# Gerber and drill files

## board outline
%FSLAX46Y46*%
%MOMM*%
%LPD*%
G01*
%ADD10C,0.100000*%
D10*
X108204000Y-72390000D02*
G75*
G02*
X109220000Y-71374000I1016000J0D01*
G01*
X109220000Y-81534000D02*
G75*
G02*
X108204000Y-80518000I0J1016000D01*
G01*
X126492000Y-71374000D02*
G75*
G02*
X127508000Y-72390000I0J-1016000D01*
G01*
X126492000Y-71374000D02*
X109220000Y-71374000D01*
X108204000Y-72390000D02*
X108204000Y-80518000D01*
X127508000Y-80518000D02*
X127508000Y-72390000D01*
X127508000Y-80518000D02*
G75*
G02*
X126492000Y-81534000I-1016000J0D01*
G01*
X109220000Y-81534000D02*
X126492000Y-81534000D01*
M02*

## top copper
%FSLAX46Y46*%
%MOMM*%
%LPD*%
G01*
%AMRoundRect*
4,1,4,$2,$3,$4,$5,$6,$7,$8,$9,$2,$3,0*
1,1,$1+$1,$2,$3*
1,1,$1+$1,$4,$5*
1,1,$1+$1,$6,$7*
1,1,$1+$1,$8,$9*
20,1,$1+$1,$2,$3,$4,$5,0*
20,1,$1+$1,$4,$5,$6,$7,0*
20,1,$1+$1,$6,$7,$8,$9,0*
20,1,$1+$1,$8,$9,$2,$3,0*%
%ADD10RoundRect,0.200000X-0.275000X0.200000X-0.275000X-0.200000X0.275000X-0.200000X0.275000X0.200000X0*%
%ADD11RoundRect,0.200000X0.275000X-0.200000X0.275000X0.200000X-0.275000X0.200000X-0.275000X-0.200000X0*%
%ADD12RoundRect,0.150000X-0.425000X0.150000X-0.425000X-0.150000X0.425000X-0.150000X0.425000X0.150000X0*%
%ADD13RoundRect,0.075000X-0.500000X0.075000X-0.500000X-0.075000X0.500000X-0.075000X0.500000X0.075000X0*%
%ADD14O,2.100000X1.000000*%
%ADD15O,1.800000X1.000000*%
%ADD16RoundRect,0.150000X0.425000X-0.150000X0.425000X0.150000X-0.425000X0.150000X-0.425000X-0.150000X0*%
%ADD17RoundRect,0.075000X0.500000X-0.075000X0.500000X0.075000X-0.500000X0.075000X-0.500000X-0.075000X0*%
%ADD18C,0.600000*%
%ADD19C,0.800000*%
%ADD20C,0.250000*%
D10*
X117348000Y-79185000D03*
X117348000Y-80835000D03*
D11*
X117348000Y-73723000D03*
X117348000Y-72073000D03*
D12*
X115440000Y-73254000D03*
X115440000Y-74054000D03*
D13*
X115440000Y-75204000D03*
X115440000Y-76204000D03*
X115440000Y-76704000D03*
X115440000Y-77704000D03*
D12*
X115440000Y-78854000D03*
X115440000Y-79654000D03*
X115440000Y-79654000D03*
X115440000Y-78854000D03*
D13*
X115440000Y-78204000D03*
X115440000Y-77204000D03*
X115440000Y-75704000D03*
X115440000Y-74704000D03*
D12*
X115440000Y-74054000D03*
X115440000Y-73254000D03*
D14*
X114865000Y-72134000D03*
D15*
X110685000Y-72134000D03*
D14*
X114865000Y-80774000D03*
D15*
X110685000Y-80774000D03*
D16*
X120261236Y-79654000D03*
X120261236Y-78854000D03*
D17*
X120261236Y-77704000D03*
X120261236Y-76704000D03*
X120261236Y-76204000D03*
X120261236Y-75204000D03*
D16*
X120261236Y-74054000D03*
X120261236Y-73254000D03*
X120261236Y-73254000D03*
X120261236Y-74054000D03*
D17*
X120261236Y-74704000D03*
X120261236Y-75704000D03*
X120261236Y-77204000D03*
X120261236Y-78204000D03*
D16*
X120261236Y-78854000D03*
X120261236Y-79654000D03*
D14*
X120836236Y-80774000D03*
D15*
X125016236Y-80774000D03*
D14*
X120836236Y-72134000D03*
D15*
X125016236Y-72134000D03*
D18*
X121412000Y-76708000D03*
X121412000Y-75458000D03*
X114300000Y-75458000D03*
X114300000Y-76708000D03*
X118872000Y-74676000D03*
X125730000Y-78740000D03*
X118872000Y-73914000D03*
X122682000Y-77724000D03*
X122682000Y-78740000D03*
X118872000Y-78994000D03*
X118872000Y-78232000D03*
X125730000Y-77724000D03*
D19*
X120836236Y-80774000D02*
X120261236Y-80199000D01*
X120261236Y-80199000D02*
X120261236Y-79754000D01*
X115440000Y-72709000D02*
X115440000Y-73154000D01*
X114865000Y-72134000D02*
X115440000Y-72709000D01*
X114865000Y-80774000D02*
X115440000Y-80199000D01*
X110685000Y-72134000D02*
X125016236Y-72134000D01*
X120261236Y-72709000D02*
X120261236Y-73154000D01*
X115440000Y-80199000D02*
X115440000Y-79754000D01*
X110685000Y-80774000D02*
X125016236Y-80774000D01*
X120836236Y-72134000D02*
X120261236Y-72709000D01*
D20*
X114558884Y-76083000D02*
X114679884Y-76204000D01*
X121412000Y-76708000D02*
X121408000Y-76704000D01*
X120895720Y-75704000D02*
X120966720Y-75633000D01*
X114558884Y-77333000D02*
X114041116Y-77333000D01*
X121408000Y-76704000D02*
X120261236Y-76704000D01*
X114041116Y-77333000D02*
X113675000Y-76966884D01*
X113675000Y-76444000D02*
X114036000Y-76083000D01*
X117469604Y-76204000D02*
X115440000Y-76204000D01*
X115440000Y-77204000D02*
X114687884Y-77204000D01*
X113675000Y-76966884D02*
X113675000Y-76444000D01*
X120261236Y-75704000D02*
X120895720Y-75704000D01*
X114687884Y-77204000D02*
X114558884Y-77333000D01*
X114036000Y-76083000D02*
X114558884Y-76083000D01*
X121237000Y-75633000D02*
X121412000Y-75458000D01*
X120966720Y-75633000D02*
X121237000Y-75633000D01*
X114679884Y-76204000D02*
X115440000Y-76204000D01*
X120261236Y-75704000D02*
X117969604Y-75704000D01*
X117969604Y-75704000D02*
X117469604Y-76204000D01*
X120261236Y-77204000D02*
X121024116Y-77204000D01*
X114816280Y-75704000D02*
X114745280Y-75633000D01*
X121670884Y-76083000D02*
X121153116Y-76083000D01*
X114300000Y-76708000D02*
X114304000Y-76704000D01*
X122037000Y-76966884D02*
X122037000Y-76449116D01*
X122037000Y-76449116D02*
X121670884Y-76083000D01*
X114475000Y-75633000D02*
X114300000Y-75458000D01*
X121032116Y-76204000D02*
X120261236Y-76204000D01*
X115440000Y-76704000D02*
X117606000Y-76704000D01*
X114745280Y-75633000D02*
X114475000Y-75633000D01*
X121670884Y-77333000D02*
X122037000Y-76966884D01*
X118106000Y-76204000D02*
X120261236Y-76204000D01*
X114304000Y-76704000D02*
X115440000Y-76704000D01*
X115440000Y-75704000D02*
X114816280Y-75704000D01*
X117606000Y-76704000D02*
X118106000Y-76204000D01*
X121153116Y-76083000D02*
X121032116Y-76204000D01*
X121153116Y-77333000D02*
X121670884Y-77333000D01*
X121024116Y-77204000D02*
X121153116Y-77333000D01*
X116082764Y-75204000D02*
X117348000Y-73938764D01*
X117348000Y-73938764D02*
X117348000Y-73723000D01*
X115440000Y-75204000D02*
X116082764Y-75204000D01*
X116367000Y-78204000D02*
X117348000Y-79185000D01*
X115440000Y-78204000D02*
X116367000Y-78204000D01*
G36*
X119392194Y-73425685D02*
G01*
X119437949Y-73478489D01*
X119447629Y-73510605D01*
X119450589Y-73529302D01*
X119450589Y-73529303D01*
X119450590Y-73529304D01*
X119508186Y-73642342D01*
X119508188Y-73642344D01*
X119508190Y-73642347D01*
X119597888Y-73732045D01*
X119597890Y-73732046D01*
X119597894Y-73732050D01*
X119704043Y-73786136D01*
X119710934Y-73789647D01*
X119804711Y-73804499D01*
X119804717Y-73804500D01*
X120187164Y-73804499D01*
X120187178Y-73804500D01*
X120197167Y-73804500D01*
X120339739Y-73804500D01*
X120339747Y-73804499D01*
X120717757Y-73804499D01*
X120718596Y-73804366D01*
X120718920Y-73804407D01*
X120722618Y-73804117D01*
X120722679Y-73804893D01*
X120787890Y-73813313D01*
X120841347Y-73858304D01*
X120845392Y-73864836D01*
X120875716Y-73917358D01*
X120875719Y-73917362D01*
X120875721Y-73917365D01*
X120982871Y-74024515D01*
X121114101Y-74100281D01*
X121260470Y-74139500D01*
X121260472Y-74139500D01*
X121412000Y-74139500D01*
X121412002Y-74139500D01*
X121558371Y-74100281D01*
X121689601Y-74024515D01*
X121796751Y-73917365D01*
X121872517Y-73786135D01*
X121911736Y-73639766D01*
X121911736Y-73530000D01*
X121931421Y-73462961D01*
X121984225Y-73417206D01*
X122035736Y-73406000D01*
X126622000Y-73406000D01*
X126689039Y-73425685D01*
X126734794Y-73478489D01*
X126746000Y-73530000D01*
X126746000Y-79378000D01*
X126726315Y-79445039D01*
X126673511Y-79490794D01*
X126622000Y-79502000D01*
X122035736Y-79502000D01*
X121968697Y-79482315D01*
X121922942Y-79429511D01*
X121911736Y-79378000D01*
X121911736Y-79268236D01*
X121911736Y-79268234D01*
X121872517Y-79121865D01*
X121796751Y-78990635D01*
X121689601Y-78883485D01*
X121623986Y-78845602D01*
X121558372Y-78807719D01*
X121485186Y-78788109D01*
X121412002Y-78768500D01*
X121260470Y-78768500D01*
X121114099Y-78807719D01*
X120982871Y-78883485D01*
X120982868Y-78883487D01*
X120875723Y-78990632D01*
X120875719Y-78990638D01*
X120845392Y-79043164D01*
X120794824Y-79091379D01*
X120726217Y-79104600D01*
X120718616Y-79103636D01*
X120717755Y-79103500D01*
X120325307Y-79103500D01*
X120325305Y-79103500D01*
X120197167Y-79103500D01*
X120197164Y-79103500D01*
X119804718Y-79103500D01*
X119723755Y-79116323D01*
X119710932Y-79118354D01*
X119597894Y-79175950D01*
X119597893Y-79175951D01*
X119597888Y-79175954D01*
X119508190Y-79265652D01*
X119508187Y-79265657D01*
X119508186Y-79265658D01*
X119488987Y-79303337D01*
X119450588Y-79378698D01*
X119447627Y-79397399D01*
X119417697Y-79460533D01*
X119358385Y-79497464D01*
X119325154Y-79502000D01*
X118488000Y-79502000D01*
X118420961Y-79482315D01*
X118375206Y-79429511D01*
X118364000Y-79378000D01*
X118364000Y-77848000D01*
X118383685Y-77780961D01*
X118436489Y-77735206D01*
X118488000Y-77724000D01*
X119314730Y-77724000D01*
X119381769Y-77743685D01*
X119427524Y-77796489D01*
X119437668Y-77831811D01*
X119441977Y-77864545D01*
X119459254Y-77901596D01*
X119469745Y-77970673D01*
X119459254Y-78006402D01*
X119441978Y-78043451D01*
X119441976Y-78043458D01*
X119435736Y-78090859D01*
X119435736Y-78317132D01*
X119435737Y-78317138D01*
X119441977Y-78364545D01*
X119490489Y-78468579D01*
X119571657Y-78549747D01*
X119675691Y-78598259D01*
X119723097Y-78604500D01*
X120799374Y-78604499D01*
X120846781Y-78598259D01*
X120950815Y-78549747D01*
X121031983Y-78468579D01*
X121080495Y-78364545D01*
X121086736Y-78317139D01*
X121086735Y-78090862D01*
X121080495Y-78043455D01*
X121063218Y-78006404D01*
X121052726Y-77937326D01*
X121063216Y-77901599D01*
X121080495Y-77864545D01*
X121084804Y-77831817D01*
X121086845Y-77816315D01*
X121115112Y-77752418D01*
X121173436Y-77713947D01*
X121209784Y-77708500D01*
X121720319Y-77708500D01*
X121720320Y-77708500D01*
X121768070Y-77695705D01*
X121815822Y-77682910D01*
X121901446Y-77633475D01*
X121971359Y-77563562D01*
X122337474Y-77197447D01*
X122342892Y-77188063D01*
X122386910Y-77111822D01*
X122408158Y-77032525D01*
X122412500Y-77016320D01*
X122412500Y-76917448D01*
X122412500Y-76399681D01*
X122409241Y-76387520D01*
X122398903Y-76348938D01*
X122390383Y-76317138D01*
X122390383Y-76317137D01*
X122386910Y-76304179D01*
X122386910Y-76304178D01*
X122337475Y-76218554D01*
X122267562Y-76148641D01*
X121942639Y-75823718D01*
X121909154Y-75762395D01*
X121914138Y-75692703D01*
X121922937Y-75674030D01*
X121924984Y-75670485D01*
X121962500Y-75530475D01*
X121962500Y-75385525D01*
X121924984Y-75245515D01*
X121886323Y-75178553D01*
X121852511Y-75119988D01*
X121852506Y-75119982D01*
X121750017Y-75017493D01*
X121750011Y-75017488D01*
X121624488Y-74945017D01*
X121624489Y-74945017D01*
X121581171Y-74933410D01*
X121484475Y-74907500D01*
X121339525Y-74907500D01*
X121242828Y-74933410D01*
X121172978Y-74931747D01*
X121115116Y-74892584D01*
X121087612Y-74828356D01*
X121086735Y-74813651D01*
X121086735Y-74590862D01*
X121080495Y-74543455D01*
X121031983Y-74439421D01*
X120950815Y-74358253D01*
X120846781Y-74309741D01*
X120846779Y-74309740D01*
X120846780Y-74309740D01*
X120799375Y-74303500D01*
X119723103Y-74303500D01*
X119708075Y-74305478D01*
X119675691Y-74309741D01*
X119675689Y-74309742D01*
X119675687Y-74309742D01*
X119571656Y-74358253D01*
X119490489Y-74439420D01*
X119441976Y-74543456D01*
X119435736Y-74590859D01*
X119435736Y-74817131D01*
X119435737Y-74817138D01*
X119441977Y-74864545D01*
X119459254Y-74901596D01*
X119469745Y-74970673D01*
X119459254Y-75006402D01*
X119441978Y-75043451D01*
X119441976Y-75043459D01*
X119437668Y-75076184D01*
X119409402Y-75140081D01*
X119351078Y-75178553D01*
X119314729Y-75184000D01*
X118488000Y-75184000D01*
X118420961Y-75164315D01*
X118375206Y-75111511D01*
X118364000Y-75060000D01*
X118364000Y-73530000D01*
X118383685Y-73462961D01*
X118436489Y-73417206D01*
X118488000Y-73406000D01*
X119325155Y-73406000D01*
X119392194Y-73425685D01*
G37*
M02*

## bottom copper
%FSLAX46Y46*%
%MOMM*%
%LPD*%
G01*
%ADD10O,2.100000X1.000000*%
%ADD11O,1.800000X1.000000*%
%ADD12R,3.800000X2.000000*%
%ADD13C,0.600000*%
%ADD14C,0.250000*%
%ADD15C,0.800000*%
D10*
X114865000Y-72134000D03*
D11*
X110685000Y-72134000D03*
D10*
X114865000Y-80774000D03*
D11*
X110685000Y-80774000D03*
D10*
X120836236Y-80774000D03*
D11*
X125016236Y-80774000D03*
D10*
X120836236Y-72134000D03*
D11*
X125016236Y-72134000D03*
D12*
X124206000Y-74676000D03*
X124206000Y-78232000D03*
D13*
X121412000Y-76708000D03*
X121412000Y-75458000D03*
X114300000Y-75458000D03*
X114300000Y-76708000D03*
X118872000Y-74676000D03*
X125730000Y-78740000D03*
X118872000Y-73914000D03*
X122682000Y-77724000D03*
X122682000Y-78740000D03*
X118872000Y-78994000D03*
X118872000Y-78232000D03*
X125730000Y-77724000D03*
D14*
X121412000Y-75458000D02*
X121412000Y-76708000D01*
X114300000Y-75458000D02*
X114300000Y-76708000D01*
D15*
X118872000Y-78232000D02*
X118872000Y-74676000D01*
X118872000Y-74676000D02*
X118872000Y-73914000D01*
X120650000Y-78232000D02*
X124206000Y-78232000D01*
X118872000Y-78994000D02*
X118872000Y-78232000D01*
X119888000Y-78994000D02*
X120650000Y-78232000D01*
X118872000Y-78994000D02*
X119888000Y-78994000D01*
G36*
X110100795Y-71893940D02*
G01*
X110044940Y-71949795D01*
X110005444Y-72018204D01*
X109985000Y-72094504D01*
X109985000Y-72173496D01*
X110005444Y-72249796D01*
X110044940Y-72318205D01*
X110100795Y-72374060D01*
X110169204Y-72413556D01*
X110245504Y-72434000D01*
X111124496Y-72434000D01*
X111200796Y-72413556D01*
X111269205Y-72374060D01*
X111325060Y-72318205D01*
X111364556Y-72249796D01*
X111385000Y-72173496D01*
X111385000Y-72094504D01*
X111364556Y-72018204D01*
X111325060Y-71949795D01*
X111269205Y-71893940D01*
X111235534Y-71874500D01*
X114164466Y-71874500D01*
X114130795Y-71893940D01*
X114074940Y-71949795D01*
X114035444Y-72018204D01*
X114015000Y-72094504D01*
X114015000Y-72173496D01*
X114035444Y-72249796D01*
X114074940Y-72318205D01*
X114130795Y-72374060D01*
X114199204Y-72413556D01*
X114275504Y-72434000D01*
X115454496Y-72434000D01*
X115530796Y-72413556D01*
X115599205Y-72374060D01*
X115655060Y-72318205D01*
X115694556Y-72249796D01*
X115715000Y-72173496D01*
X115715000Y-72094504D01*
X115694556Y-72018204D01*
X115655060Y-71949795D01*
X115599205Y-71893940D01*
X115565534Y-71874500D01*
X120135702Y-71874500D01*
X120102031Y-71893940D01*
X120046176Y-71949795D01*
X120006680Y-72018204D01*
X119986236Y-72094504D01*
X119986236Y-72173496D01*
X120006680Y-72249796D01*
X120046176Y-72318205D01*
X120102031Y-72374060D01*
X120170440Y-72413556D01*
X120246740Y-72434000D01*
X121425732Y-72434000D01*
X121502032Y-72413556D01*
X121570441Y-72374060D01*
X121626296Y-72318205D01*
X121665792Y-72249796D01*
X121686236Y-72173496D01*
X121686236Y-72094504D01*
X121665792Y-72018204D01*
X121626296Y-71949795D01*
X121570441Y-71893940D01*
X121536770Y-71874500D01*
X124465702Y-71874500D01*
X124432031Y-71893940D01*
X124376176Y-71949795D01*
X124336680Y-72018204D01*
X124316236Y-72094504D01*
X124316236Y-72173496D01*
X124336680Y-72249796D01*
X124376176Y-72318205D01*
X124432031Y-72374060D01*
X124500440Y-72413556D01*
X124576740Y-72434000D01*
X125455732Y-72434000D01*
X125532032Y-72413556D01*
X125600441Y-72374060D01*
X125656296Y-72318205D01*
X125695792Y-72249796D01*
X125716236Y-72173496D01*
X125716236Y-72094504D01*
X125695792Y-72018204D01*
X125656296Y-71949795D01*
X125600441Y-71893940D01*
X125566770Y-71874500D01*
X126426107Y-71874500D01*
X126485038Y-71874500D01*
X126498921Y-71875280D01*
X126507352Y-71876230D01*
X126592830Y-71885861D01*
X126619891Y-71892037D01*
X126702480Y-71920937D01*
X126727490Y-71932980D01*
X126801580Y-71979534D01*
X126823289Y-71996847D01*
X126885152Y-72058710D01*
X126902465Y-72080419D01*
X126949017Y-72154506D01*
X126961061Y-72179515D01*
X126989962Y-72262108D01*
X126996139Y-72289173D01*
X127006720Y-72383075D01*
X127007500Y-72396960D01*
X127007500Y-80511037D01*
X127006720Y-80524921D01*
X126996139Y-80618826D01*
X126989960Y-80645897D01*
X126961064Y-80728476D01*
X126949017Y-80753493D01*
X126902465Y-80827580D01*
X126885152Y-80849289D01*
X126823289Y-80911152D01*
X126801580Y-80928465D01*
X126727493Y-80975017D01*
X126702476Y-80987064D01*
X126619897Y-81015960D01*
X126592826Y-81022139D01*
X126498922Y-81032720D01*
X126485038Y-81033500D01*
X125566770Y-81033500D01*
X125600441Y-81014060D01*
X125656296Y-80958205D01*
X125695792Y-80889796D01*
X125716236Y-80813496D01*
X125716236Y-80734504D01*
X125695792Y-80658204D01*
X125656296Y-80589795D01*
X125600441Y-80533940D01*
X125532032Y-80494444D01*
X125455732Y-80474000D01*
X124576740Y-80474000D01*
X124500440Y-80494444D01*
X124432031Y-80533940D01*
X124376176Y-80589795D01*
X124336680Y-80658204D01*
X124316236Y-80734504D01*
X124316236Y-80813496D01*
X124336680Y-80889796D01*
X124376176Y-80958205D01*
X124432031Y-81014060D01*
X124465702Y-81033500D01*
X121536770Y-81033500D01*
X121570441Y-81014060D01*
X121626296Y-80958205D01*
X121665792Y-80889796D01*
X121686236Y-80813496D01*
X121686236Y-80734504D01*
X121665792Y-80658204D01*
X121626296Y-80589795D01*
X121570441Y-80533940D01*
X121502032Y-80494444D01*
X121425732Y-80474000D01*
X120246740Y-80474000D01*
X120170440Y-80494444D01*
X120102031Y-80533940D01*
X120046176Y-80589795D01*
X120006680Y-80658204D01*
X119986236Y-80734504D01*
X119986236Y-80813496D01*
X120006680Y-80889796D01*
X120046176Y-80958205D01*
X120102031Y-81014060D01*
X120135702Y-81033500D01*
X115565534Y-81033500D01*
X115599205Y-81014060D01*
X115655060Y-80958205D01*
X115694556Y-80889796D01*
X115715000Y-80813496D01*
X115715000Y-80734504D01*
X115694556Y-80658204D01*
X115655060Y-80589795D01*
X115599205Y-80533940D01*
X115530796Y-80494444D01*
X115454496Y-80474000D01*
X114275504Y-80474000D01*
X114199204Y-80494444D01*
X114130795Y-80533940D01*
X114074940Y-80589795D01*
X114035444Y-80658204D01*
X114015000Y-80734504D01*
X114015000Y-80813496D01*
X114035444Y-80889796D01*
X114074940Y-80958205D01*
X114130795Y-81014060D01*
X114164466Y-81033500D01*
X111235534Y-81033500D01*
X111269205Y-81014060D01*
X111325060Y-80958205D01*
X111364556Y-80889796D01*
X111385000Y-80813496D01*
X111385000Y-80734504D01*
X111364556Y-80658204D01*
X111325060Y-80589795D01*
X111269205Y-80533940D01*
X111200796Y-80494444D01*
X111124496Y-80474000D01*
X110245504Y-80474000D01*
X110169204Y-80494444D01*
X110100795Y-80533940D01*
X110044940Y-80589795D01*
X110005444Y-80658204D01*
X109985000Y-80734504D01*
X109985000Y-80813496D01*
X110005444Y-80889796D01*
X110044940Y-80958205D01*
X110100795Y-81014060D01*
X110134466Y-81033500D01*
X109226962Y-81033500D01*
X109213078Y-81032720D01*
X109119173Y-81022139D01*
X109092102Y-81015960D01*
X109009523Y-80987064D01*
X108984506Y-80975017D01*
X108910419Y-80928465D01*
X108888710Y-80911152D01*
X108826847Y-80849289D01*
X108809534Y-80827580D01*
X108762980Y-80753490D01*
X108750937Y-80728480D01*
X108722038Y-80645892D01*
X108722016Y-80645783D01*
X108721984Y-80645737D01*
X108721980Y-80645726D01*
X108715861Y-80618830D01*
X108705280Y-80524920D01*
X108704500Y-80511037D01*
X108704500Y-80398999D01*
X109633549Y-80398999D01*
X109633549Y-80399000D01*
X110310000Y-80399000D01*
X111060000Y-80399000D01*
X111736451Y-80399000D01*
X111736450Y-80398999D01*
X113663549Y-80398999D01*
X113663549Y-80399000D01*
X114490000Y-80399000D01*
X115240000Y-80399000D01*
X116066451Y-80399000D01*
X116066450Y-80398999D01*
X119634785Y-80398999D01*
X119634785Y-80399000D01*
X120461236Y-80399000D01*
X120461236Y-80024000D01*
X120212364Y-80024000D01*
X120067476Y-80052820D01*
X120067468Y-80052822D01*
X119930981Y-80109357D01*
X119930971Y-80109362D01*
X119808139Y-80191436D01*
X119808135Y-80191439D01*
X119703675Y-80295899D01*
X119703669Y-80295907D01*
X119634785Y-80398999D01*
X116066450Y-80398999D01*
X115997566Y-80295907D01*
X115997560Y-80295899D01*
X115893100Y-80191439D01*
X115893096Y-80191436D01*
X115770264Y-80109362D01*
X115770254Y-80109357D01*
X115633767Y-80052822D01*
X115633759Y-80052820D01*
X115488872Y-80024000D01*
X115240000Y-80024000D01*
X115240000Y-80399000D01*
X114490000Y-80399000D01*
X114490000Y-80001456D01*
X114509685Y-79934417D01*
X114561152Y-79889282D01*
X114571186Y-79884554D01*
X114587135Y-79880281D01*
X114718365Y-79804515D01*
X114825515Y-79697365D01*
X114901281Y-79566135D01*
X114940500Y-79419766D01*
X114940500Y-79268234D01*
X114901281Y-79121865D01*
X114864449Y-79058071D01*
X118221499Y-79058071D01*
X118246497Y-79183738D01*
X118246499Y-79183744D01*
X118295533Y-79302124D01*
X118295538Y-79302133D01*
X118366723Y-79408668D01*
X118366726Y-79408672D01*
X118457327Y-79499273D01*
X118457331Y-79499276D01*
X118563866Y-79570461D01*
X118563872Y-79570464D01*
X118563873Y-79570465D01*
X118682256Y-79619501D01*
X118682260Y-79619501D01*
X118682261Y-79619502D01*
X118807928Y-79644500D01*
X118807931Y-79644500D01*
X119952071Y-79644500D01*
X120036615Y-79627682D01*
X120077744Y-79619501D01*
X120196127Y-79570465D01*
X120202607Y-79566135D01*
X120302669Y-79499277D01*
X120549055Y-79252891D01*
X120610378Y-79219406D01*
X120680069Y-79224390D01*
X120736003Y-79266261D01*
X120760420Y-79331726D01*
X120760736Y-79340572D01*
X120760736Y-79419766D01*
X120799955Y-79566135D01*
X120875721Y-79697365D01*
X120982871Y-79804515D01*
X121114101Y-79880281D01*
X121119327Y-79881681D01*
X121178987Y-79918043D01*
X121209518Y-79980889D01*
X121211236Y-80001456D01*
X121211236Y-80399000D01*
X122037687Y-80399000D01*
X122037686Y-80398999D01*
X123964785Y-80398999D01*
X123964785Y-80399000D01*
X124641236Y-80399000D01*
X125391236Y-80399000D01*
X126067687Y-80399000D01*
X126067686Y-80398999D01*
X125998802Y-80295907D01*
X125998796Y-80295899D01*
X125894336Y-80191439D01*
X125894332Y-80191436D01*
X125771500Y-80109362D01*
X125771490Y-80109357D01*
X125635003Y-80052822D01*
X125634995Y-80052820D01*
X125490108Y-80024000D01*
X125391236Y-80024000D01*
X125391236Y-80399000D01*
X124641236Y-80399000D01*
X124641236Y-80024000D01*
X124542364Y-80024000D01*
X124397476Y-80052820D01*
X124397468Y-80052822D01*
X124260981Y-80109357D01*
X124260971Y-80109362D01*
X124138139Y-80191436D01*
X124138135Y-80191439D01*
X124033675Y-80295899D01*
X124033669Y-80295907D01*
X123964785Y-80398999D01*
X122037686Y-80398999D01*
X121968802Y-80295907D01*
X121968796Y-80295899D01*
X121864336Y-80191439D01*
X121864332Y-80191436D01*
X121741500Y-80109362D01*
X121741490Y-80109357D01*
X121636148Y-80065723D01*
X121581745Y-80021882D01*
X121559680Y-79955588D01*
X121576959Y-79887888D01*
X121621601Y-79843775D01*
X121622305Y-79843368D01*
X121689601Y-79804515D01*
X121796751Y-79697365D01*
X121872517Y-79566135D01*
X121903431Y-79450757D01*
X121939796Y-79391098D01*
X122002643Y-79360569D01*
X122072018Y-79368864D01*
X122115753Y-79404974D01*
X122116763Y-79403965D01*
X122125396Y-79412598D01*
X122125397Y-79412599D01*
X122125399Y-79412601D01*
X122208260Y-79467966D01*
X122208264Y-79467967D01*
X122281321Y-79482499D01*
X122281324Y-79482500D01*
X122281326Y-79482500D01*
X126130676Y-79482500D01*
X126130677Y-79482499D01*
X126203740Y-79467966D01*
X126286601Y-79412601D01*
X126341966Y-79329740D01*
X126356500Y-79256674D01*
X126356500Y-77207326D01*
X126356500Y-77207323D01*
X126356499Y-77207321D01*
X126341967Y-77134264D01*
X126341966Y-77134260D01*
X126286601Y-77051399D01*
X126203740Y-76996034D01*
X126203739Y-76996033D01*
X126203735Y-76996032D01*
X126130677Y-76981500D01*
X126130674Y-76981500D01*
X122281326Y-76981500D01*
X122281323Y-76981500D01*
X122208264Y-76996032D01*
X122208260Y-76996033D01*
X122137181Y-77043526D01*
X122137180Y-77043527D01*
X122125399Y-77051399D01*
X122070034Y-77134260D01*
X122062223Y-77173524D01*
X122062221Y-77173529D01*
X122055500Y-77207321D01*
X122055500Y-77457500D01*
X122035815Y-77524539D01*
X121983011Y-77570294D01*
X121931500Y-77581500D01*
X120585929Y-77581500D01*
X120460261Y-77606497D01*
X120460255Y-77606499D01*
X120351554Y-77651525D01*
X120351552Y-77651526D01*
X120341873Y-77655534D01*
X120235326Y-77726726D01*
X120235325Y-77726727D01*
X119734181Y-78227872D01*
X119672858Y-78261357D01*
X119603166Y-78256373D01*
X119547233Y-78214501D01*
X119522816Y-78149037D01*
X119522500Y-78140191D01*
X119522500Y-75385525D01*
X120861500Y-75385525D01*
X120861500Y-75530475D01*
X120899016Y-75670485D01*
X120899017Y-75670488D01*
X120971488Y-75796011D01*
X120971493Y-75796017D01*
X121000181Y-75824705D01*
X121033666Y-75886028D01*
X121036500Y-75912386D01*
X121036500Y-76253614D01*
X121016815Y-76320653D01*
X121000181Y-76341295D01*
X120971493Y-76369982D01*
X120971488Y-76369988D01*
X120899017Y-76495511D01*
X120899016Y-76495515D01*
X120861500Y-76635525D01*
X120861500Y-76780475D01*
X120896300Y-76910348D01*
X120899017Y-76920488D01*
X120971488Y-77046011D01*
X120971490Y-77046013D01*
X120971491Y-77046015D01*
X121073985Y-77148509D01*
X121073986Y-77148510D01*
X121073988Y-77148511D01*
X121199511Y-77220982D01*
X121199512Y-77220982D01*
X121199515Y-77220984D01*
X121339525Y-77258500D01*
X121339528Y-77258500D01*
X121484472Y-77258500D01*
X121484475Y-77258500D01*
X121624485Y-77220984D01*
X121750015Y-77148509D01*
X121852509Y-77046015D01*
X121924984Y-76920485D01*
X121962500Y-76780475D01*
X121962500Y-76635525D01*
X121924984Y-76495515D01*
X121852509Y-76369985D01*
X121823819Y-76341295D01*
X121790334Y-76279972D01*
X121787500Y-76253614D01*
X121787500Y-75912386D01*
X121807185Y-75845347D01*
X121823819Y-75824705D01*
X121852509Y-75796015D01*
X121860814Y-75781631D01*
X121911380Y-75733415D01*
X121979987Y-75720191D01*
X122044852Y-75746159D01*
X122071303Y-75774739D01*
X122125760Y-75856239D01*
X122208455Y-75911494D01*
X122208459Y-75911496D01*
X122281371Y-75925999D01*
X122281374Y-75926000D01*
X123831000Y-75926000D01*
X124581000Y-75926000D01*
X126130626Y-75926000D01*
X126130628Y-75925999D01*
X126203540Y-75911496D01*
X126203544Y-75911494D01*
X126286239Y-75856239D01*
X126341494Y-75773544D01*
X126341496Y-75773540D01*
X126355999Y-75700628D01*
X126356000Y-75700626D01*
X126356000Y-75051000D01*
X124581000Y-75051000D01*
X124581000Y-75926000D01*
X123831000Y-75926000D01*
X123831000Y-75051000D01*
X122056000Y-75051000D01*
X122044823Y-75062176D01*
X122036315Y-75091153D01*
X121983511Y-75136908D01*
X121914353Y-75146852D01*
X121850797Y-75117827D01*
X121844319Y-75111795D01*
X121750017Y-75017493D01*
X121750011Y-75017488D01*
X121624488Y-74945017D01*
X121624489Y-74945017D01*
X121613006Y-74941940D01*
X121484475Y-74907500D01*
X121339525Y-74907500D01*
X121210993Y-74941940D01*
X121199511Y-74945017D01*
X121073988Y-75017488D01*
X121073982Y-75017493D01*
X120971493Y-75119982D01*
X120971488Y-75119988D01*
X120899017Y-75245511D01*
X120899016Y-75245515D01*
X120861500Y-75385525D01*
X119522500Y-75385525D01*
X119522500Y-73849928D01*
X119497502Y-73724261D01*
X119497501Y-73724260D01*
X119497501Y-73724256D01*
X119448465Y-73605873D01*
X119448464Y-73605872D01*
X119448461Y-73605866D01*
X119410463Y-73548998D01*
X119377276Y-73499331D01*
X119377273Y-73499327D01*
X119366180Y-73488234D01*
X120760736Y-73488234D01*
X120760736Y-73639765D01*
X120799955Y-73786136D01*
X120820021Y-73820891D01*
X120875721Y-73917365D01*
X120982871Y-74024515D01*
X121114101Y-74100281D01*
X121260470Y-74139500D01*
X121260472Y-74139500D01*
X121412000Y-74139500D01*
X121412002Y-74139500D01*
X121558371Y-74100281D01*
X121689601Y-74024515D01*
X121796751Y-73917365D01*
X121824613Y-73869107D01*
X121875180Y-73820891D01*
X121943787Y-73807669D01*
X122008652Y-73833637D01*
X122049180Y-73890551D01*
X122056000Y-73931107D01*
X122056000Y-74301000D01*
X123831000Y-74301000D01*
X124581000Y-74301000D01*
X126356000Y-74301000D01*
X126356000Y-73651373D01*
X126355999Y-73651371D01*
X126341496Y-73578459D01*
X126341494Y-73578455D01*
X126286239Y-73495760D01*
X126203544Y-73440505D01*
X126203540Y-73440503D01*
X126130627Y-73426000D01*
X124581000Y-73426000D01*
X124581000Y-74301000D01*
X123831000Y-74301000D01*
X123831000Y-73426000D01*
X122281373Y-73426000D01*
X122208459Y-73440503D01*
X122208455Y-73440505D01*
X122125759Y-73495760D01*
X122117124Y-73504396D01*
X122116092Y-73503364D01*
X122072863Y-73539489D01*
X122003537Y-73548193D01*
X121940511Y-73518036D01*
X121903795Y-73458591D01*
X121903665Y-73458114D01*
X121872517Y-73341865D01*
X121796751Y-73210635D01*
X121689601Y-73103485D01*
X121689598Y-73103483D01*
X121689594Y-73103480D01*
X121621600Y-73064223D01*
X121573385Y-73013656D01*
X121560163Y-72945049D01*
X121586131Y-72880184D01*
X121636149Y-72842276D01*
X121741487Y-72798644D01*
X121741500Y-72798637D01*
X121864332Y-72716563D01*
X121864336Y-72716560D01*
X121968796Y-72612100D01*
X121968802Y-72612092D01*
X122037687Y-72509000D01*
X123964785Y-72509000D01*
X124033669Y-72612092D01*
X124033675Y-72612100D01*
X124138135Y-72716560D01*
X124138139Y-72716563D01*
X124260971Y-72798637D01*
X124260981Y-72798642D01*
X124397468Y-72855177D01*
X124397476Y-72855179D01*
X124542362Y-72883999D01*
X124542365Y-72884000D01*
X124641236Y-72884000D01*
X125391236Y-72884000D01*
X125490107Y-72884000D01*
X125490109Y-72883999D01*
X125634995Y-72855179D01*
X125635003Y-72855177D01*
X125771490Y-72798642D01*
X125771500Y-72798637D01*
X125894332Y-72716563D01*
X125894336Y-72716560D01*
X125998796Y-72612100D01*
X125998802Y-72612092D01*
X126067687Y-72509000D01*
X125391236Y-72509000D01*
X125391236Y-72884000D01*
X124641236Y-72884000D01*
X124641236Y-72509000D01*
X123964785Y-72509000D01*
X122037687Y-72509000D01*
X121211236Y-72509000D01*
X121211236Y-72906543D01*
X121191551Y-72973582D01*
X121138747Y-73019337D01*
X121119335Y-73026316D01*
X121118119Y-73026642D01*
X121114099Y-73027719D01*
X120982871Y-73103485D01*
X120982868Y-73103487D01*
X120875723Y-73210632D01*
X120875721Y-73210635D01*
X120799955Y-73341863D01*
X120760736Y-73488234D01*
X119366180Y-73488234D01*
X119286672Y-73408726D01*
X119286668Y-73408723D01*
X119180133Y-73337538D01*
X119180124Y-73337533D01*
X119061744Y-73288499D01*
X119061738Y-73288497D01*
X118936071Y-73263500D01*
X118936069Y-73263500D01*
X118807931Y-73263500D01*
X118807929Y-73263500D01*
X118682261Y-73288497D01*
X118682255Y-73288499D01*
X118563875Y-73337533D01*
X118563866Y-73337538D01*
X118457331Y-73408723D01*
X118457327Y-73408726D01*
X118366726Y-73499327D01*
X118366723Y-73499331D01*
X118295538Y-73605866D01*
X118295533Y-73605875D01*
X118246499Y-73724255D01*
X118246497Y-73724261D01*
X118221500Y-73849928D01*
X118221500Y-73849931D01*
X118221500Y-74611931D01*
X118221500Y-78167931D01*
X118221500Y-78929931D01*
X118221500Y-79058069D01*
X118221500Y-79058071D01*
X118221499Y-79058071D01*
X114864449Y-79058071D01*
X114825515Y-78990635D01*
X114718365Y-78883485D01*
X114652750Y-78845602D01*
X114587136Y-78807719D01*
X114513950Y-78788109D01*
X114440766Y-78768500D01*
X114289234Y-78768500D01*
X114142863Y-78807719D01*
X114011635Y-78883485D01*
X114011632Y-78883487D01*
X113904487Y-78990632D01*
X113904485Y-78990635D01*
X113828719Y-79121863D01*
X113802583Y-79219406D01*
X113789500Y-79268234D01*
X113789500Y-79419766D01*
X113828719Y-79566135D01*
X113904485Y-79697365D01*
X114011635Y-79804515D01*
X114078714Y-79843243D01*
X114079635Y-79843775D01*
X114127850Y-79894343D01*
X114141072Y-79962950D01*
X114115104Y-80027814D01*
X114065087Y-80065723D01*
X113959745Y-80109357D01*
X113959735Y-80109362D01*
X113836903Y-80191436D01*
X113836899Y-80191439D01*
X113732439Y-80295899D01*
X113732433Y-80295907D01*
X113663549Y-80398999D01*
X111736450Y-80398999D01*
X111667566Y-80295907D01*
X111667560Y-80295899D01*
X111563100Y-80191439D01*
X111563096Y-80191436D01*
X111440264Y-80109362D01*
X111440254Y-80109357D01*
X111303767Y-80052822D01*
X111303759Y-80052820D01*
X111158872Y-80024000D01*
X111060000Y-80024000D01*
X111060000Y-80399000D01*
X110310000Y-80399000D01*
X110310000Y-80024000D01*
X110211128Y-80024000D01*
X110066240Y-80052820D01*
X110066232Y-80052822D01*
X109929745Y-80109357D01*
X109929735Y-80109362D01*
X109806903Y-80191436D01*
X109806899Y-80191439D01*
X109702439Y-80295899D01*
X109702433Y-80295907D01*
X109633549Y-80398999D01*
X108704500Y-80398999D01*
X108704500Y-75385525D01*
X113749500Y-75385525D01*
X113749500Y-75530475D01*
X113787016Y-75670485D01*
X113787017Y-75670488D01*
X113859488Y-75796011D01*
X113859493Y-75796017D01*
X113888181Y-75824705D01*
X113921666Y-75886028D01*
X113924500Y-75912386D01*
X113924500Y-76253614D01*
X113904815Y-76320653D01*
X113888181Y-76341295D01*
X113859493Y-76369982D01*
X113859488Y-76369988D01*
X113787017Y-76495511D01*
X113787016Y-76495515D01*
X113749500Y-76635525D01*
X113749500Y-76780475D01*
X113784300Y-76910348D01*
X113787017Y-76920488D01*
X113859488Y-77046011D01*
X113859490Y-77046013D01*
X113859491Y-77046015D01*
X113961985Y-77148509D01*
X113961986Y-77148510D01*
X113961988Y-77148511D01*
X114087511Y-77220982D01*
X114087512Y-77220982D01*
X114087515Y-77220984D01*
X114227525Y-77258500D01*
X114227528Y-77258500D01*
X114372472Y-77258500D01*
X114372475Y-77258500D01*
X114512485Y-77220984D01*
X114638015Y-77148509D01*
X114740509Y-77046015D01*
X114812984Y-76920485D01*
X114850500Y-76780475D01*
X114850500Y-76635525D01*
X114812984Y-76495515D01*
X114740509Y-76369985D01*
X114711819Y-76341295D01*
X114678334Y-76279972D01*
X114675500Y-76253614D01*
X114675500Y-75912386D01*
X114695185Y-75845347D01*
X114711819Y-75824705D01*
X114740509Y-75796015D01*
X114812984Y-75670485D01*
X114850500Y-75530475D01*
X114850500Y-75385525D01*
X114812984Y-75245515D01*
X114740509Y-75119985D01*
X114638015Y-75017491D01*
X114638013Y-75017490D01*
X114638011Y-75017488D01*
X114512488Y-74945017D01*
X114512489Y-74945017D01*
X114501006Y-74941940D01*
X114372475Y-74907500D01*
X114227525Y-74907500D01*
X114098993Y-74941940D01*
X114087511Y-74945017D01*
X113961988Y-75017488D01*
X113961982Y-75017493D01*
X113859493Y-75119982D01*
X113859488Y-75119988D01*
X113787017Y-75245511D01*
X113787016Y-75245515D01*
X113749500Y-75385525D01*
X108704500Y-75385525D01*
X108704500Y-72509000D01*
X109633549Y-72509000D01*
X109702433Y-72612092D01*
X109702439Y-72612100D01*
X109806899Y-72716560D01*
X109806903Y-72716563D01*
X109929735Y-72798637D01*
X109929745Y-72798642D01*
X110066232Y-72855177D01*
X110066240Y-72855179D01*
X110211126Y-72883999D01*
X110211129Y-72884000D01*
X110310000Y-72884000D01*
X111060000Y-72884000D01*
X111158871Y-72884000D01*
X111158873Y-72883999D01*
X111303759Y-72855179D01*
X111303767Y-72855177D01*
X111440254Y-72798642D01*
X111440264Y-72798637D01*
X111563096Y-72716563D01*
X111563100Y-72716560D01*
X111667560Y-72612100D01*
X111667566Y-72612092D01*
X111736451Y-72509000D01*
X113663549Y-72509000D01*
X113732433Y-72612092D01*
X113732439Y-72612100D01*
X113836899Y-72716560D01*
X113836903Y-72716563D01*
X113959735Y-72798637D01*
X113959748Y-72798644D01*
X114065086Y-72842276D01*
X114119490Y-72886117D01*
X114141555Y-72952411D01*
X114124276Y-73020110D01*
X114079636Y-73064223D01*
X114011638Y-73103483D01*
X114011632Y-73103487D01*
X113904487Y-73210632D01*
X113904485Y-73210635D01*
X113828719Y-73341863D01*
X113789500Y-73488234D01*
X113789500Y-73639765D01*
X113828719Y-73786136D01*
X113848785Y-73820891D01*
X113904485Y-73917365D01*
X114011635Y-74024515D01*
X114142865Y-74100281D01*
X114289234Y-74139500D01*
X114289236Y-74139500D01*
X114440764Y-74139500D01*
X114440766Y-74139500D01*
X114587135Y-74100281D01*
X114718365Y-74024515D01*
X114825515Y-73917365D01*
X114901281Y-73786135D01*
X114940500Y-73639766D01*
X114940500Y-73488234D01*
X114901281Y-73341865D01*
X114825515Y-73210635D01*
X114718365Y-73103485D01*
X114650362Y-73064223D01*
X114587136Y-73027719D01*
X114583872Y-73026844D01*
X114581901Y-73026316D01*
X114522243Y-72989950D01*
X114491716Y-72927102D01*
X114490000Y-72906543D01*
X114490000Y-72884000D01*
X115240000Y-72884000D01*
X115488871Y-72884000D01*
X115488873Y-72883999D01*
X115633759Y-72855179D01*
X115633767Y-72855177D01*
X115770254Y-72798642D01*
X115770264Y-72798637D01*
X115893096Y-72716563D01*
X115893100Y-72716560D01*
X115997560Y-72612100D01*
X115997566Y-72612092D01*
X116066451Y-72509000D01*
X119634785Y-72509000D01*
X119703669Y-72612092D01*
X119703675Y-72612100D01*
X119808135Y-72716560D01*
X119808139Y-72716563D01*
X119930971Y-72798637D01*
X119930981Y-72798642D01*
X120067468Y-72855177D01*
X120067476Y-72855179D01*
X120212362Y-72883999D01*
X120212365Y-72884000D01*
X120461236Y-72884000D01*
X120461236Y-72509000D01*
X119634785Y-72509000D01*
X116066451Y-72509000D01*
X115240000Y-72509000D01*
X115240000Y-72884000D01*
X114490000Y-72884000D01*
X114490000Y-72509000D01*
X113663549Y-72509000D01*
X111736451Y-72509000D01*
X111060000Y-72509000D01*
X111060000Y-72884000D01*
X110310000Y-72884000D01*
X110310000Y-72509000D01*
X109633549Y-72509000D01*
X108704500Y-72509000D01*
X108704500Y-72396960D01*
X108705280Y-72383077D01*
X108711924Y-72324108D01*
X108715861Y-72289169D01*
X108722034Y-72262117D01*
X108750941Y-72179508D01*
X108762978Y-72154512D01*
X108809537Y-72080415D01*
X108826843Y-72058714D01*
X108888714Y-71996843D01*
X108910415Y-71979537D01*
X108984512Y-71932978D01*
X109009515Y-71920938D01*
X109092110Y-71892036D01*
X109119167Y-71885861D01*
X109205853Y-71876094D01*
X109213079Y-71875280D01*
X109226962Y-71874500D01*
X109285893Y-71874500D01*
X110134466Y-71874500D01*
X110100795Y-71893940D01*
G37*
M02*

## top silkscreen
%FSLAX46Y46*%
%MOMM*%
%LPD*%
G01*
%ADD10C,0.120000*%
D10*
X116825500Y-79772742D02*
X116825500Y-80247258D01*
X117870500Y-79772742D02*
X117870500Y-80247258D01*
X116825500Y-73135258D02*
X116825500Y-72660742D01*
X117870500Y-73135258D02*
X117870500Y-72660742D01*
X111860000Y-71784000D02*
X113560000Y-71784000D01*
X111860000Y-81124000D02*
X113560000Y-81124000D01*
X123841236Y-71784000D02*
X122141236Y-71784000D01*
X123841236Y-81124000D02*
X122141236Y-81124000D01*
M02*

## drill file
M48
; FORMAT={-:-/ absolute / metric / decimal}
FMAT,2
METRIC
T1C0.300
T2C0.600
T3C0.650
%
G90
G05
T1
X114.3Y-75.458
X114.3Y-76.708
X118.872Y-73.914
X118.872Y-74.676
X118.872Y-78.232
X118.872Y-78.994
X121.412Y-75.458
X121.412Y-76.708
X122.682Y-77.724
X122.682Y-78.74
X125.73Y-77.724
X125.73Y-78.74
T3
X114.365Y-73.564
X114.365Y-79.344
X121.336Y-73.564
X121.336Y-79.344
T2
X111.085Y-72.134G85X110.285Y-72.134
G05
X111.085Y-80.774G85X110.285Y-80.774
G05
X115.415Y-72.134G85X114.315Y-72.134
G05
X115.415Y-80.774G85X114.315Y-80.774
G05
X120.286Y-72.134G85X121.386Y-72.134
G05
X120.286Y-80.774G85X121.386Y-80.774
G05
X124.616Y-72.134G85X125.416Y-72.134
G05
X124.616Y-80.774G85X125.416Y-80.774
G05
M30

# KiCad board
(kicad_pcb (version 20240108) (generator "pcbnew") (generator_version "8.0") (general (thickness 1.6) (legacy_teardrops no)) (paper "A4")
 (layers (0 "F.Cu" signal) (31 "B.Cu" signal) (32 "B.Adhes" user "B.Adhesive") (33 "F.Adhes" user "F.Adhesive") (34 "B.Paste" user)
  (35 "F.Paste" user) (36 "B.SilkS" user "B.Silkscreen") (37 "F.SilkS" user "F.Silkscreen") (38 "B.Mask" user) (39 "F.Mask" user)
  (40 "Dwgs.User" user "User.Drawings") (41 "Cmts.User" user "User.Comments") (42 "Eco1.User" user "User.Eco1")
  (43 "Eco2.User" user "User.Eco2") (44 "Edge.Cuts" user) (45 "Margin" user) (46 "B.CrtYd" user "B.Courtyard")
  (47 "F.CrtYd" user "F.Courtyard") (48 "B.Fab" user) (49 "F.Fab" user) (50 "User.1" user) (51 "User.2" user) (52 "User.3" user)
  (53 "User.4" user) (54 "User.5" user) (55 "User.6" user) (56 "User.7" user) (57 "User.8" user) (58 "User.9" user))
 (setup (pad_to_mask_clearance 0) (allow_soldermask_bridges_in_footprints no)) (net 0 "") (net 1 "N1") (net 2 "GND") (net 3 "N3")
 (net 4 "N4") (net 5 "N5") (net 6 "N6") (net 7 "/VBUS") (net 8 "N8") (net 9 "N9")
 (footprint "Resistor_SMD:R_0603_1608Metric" (layer "F.Cu") (at 117.348 80.01 -90)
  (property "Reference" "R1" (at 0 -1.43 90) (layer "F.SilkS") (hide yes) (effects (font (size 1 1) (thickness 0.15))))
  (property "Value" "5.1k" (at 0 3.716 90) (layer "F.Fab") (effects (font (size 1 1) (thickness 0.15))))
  (fp_line (start -0.237258 0.5225) (end 0.237258 0.5225) (stroke (width 0.12) (type solid)) (layer "F.SilkS"))
  (fp_line (start -0.237258 -0.5225) (end 0.237258 -0.5225) (stroke (width 0.12) (type solid)) (layer "F.SilkS"))
  (pad "1" smd roundrect (at -0.825 0 270) (size 0.8 0.95) (layers "F.Cu" "F.Paste" "F.Mask") (roundrect_rratio 0.25) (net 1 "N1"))
  (pad "2" smd roundrect (at 0.825 0 270) (size 0.8 0.95) (layers "F.Cu" "F.Paste" "F.Mask") (roundrect_rratio 0.25) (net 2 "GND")))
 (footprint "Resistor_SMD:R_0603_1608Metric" (layer "F.Cu") (at 117.348 72.898 90)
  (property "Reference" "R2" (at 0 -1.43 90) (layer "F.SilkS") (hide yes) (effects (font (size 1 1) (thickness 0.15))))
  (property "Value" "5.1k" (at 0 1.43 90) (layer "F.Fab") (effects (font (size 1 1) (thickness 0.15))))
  (fp_line (start -0.237258 -0.5225) (end 0.237258 -0.5225) (stroke (width 0.12) (type solid)) (layer "F.SilkS"))
  (fp_line (start -0.237258 0.5225) (end 0.237258 0.5225) (stroke (width 0.12) (type solid)) (layer "F.SilkS"))
  (pad "1" smd roundrect (at -0.825 0 90) (size 0.8 0.95) (layers "F.Cu" "F.Paste" "F.Mask") (roundrect_rratio 0.25) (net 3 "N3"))
  (pad "2" smd roundrect (at 0.825 0 90) (size 0.8 0.95) (layers "F.Cu" "F.Paste" "F.Mask") (roundrect_rratio 0.25) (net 2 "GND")))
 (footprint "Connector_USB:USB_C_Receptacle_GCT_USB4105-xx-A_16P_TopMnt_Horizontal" (layer "F.Cu") (at 111.76 76.454 -90)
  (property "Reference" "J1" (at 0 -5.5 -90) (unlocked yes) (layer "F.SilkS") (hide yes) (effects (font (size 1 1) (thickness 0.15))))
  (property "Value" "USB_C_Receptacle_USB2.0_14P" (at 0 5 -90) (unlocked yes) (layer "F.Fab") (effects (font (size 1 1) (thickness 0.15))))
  (fp_line (start -4.67 -0.1) (end -4.67 -1.8) (stroke (width 0.12) (type solid)) (layer "F.SilkS"))
  (fp_line (start 4.67 -0.1) (end 4.67 -1.8) (stroke (width 0.12) (type solid)) (layer "F.SilkS"))
  (pad "" np_thru_hole circle (at -2.89 -2.605 270) (size 0.65 0.65) (drill 0.65) (layers "F&B.Cu" "*.Mask"))
  (pad "" np_thru_hole circle (at 2.89 -2.605 270) (size 0.65 0.65) (drill 0.65) (layers "F&B.Cu" "*.Mask"))
  (pad "A1" smd roundrect (at -3.2 -3.68 270) (size 0.6 1.15) (layers "F.Cu" "F.Paste" "F.Mask") (roundrect_rratio 0.25) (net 2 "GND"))
  (pad "A4" smd roundrect (at -2.4 -3.68 270) (size 0.6 1.15) (layers "F.Cu" "F.Paste" "F.Mask") (roundrect_rratio 0.25) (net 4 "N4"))
  (pad "A5" smd roundrect (at -1.25 -3.68 270) (size 0.3 1.15) (layers "F.Cu" "F.Paste" "F.Mask") (roundrect_rratio 0.25) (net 3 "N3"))
  (pad "A6" smd roundrect (at -0.25 -3.68 270) (size 0.3 1.15) (layers "F.Cu" "F.Paste" "F.Mask") (roundrect_rratio 0.25) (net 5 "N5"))
  (pad "A7" smd roundrect (at 0.25 -3.68 270) (size 0.3 1.15) (layers "F.Cu" "F.Paste" "F.Mask") (roundrect_rratio 0.25) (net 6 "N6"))
  (pad "A8" smd roundrect (at 1.25 -3.68 270) (size 0.3 1.15) (layers "F.Cu" "F.Paste" "F.Mask") (roundrect_rratio 0.25))
  (pad "A9" smd roundrect (at 2.4 -3.68 270) (size 0.6 1.15) (layers "F.Cu" "F.Paste" "F.Mask") (roundrect_rratio 0.25) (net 4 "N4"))
  (pad "A12" smd roundrect (at 3.2 -3.68 270) (size 0.6 1.15) (layers "F.Cu" "F.Paste" "F.Mask") (roundrect_rratio 0.25) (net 2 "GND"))
  (pad "B1" smd roundrect (at 3.2 -3.68 270) (size 0.6 1.15) (layers "F.Cu" "F.Paste" "F.Mask") (roundrect_rratio 0.25) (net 2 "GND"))
  (pad "B4" smd roundrect (at 2.4 -3.68 270) (size 0.6 1.15) (layers "F.Cu" "F.Paste" "F.Mask") (roundrect_rratio 0.25) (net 4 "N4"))
  (pad "B5" smd roundrect (at 1.75 -3.68 270) (size 0.3 1.15) (layers "F.Cu" "F.Paste" "F.Mask") (roundrect_rratio 0.25) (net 1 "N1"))
  (pad "B6" smd roundrect (at 0.75 -3.68 270) (size 0.3 1.15) (layers "F.Cu" "F.Paste" "F.Mask") (roundrect_rratio 0.25) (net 5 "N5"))
  (pad "B7" smd roundrect (at -0.75 -3.68 270) (size 0.3 1.15) (layers "F.Cu" "F.Paste" "F.Mask") (roundrect_rratio 0.25) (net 6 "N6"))
  (pad "B8" smd roundrect (at -1.75 -3.68 270) (size 0.3 1.15) (layers "F.Cu" "F.Paste" "F.Mask") (roundrect_rratio 0.25))
  (pad "B9" smd roundrect (at -2.4 -3.68 270) (size 0.6 1.15) (layers "F.Cu" "F.Paste" "F.Mask") (roundrect_rratio 0.25) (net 4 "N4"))
  (pad "B12" smd roundrect (at -3.2 -3.68 270) (size 0.6 1.15) (layers "F.Cu" "F.Paste" "F.Mask") (roundrect_rratio 0.25) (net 2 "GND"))
  (pad "S1" thru_hole oval (at -4.32 -3.105 270) (size 1 2.1) (drill oval 0.6 1.7) (layers "*.Cu" "*.Mask" "F.Paste")
   (remove_unused_layers no) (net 2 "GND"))
  (pad "S1" thru_hole oval (at -4.32 1.075 270) (size 1 1.8) (drill oval 0.6 1.4) (layers "*.Cu" "*.Mask" "F.Paste")
   (remove_unused_layers no) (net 2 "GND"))
  (pad "S1" thru_hole oval (at 4.32 -3.105 270) (size 1 2.1) (drill oval 0.6 1.7) (layers "*.Cu" "*.Mask" "F.Paste")
   (remove_unused_layers no) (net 2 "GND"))
  (pad "S1" thru_hole oval (at 4.32 1.075 270) (size 1 1.8) (drill oval 0.6 1.4) (layers "*.Cu" "*.Mask" "F.Paste")
   (remove_unused_layers no) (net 2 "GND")))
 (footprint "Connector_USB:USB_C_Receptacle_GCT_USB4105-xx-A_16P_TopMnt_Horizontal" (layer "F.Cu") (at 123.941236 76.454 90)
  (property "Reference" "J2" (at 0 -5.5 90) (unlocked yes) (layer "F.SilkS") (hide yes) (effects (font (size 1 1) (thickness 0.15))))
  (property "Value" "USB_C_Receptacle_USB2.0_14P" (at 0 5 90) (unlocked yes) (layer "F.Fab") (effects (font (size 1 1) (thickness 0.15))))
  (fp_line (start 4.67 -0.1) (end 4.67 -1.8) (stroke (width 0.12) (type solid)) (layer "F.SilkS"))
  (fp_line (start -4.67 -0.1) (end -4.67 -1.8) (stroke (width 0.12) (type solid)) (layer "F.SilkS"))
  (pad "" np_thru_hole circle (at -2.89 -2.605 90) (size 0.65 0.65) (drill 0.65) (layers "F&B.Cu" "*.Mask"))
  (pad "" np_thru_hole circle (at 2.89 -2.605 90) (size 0.65 0.65) (drill 0.65) (layers "F&B.Cu" "*.Mask"))
  (pad "A1" smd roundrect (at -3.2 -3.68 90) (size 0.6 1.15) (layers "F.Cu" "F.Paste" "F.Mask") (roundrect_rratio 0.25) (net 2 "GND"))
  (pad "A4" smd roundrect (at -2.4 -3.68 90) (size 0.6 1.15) (layers "F.Cu" "F.Paste" "F.Mask") (roundrect_rratio 0.25) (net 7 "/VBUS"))
  (pad "A5" smd roundrect (at -1.25 -3.68 90) (size 0.3 1.15) (layers "F.Cu" "F.Paste" "F.Mask") (roundrect_rratio 0.25) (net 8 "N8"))
  (pad "A6" smd roundrect (at -0.25 -3.68 90) (size 0.3 1.15) (layers "F.Cu" "F.Paste" "F.Mask") (roundrect_rratio 0.25) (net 5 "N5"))
  (pad "A7" smd roundrect (at 0.25 -3.68 90) (size 0.3 1.15) (layers "F.Cu" "F.Paste" "F.Mask") (roundrect_rratio 0.25) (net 6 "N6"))
  (pad "A8" smd roundrect (at 1.25 -3.68 90) (size 0.3 1.15) (layers "F.Cu" "F.Paste" "F.Mask") (roundrect_rratio 0.25))
  (pad "A9" smd roundrect (at 2.4 -3.68 90) (size 0.6 1.15) (layers "F.Cu" "F.Paste" "F.Mask") (roundrect_rratio 0.25) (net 7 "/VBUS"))
  (pad "A12" smd roundrect (at 3.2 -3.68 90) (size 0.6 1.15) (layers "F.Cu" "F.Paste" "F.Mask") (roundrect_rratio 0.25) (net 2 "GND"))
  (pad "B1" smd roundrect (at 3.2 -3.68 90) (size 0.6 1.15) (layers "F.Cu" "F.Paste" "F.Mask") (roundrect_rratio 0.25) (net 2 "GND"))
  (pad "B4" smd roundrect (at 2.4 -3.68 90) (size 0.6 1.15) (layers "F.Cu" "F.Paste" "F.Mask") (roundrect_rratio 0.25) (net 7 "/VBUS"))
  (pad "B5" smd roundrect (at 1.75 -3.68 90) (size 0.3 1.15) (layers "F.Cu" "F.Paste" "F.Mask") (roundrect_rratio 0.25) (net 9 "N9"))
  (pad "B6" smd roundrect (at 0.75 -3.68 90) (size 0.3 1.15) (layers "F.Cu" "F.Paste" "F.Mask") (roundrect_rratio 0.25) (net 5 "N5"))
  (pad "B7" smd roundrect (at -0.75 -3.68 90) (size 0.3 1.15) (layers "F.Cu" "F.Paste" "F.Mask") (roundrect_rratio 0.25) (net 6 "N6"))
  (pad "B8" smd roundrect (at -1.75 -3.68 90) (size 0.3 1.15) (layers "F.Cu" "F.Paste" "F.Mask") (roundrect_rratio 0.25))
  (pad "B9" smd roundrect (at -2.4 -3.68 90) (size 0.6 1.15) (layers "F.Cu" "F.Paste" "F.Mask") (roundrect_rratio 0.25) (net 7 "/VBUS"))
  (pad "B12" smd roundrect (at -3.2 -3.68 90) (size 0.6 1.15) (layers "F.Cu" "F.Paste" "F.Mask") (roundrect_rratio 0.25) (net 2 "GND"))
  (pad "S1" thru_hole oval (at -4.32 -3.105 90) (size 1 2.1) (drill oval 0.6 1.7) (layers "*.Cu" "*.Mask" "F.Paste")
   (remove_unused_layers no) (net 2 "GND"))
  (pad "S1" thru_hole oval (at -4.32 1.075 90) (size 1 1.8) (drill oval 0.6 1.4) (layers "*.Cu" "*.Mask" "F.Paste")
   (remove_unused_layers no) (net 2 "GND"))
  (pad "S1" thru_hole oval (at 4.32 -3.105 90) (size 1 2.1) (drill oval 0.6 1.7) (layers "*.Cu" "*.Mask" "F.Paste")
   (remove_unused_layers no) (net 2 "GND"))
  (pad "S1" thru_hole oval (at 4.32 1.075 90) (size 1 1.8) (drill oval 0.6 1.4) (layers "*.Cu" "*.Mask" "F.Paste") (remove_unused_layers no)
   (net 2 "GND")))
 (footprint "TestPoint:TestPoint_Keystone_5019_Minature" (layer "B.Cu") (at 124.206 74.676 180)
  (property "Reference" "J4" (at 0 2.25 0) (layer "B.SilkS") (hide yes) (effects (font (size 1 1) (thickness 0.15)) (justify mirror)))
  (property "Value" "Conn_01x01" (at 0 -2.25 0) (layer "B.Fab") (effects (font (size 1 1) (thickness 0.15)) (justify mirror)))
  (pad "1" smd rect (at 0 0 180) (size 3.8 2) (layers "B.Cu" "B.Paste" "B.Mask") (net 2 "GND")))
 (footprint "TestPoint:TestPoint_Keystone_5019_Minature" (layer "B.Cu") (at 124.206 78.232 180)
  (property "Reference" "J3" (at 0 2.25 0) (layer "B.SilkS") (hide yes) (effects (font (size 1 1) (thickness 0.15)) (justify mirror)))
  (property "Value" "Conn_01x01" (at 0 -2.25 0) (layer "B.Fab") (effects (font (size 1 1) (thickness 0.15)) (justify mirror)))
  (pad "1" smd rect (at 0 0 180) (size 3.8 2) (layers "B.Cu" "B.Paste" "B.Mask") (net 7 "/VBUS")))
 (gr_arc (start 108.204 72.39) (mid 108.50158 71.67158) (end 109.22 71.374) (stroke (width 0.1) (type default)) (layer "Edge.Cuts"))
 (gr_arc (start 109.22 81.534) (mid 108.50158 81.23642) (end 108.204 80.518) (stroke (width 0.1) (type default)) (layer "Edge.Cuts"))
 (gr_arc (start 126.492 71.374) (mid 127.21042 71.67158) (end 127.508 72.39) (stroke (width 0.1) (type default)) (layer "Edge.Cuts"))
 (gr_line (start 126.492 71.374) (end 109.22 71.374) (stroke (width 0.1) (type default)) (layer "Edge.Cuts"))
 (gr_line (start 108.204 72.39) (end 108.204 80.518) (stroke (width 0.1) (type default)) (layer "Edge.Cuts"))
 (gr_line (start 127.508 80.518) (end 127.508 72.39) (stroke (width 0.1) (type default)) (layer "Edge.Cuts"))
 (gr_arc (start 127.508 80.518) (mid 127.21042 81.23642) (end 126.492 81.534) (stroke (width 0.1) (type default)) (layer "Edge.Cuts"))
 (gr_line (start 109.22 81.534) (end 126.492 81.534) (stroke (width 0.1) (type default)) (layer "Edge.Cuts"))
 (segment (start 120.836236 80.774) (end 120.261236 80.199) (width 0.8) (layer "F.Cu") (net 2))
 (segment (start 120.261236 80.199) (end 120.261236 79.754) (width 0.8) (layer "F.Cu") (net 2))
 (segment (start 115.44 72.709) (end 115.44 73.154) (width 0.8) (layer "F.Cu") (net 2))
 (segment (start 114.865 72.134) (end 115.44 72.709) (width 0.8) (layer "F.Cu") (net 2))
 (segment (start 114.865 80.774) (end 115.44 80.199) (width 0.8) (layer "F.Cu") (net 2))
 (segment (start 110.685 72.134) (end 125.016236 72.134) (width 0.8) (layer "F.Cu") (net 2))
 (segment (start 120.261236 72.709) (end 120.261236 73.154) (width 0.8) (layer "F.Cu") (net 2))
 (segment (start 115.44 80.199) (end 115.44 79.754) (width 0.8) (layer "F.Cu") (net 2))
 (segment (start 110.685 80.774) (end 125.016236 80.774) (width 0.8) (layer "F.Cu") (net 2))
 (segment (start 120.836236 72.134) (end 120.261236 72.709) (width 0.8) (layer "F.Cu") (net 2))
 (segment (start 114.558884 76.083) (end 114.679884 76.204) (width 0.25) (layer "F.Cu") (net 5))
 (segment (start 121.412 76.708) (end 121.408 76.704) (width 0.25) (layer "F.Cu") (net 5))
 (segment (start 120.89572 75.704) (end 120.96672 75.633) (width 0.25) (layer "F.Cu") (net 5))
 (segment (start 114.558884 77.333) (end 114.041116 77.333) (width 0.25) (layer "F.Cu") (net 5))
 (segment (start 121.408 76.704) (end 120.261236 76.704) (width 0.25) (layer "F.Cu") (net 5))
 (segment (start 114.041116 77.333) (end 113.675 76.966884) (width 0.25) (layer "F.Cu") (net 5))
 (segment (start 113.675 76.444) (end 114.036 76.083) (width 0.25) (layer "F.Cu") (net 5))
 (segment (start 117.469604 76.204) (end 115.44 76.204) (width 0.25) (layer "F.Cu") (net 5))
 (segment (start 115.44 77.204) (end 114.687884 77.204) (width 0.25) (layer "F.Cu") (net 5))
 (segment (start 113.675 76.966884) (end 113.675 76.444) (width 0.25) (layer "F.Cu") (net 5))
 (segment (start 120.261236 75.704) (end 120.89572 75.704) (width 0.25) (layer "F.Cu") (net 5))
 (segment (start 114.687884 77.204) (end 114.558884 77.333) (width 0.25) (layer "F.Cu") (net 5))
 (segment (start 114.036 76.083) (end 114.558884 76.083) (width 0.25) (layer "F.Cu") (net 5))
 (segment (start 121.237 75.633) (end 121.412 75.458) (width 0.25) (layer "F.Cu") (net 5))
 (segment (start 120.96672 75.633) (end 121.237 75.633) (width 0.25) (layer "F.Cu") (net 5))
 (segment (start 114.679884 76.204) (end 115.44 76.204) (width 0.25) (layer "F.Cu") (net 5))
 (segment (start 120.261236 75.704) (end 117.969604 75.704) (width 0.25) (layer "F.Cu") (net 5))
 (segment (start 117.969604 75.704) (end 117.469604 76.204) (width 0.25) (layer "F.Cu") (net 5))
 (via (at 121.412 76.708) (size 0.6) (drill 0.3) (layers "F.Cu" "B.Cu") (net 5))
 (via (at 121.412 75.458) (size 0.6) (drill 0.3) (layers "F.Cu" "B.Cu") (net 5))
 (segment (start 121.412 75.458) (end 121.412 76.708) (width 0.25) (layer "B.Cu") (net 5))
 (segment (start 120.261236 77.204) (end 121.024116 77.204) (width 0.25) (layer "F.Cu") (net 6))
 (segment (start 114.81628 75.704) (end 114.74528 75.633) (width 0.25) (layer "F.Cu") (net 6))
 (segment (start 121.670884 76.083) (end 121.153116 76.083) (width 0.25) (layer "F.Cu") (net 6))
 (segment (start 114.3 76.708) (end 114.304 76.704) (width 0.25) (layer "F.Cu") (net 6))
 (segment (start 122.037 76.966884) (end 122.037 76.449116) (width 0.25) (layer "F.Cu") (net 6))
 (segment (start 122.037 76.449116) (end 121.670884 76.083) (width 0.25) (layer "F.Cu") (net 6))
 (segment (start 114.475 75.633) (end 114.3 75.458) (width 0.25) (layer "F.Cu") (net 6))
 (segment (start 121.032116 76.204) (end 120.261236 76.204) (width 0.25) (layer "F.Cu") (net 6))
 (segment (start 115.44 76.704) (end 117.606 76.704) (width 0.25) (layer "F.Cu") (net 6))
 (segment (start 114.74528 75.633) (end 114.475 75.633) (width 0.25) (layer "F.Cu") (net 6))
 (segment (start 121.670884 77.333) (end 122.037 76.966884) (width 0.25) (layer "F.Cu") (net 6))
 (segment (start 118.106 76.204) (end 120.261236 76.204) (width 0.25) (layer "F.Cu") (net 6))
 (segment (start 114.304 76.704) (end 115.44 76.704) (width 0.25) (layer "F.Cu") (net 6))
 (segment (start 115.44 75.704) (end 114.81628 75.704) (width 0.25) (layer "F.Cu") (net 6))
 (segment (start 117.606 76.704) (end 118.106 76.204) (width 0.25) (layer "F.Cu") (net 6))
 (segment (start 121.153116 76.083) (end 121.032116 76.204) (width 0.25) (layer "F.Cu") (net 6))
 (segment (start 121.153116 77.333) (end 121.670884 77.333) (width 0.25) (layer "F.Cu") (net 6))
 (segment (start 121.024116 77.204) (end 121.153116 77.333) (width 0.25) (layer "F.Cu") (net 6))
 (via (at 114.3 75.458) (size 0.6) (drill 0.3) (layers "F.Cu" "B.Cu") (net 6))
 (via (at 114.3 76.708) (size 0.6) (drill 0.3) (layers "F.Cu" "B.Cu") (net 6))
 (segment (start 114.3 75.458) (end 114.3 76.708) (width 0.25) (layer "B.Cu") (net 6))
 (segment (start 116.082764 75.204) (end 117.348 73.938764) (width 0.25) (layer "F.Cu") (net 3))
 (segment (start 117.348 73.938764) (end 117.348 73.723) (width 0.25) (layer "F.Cu") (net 3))
 (segment (start 115.44 75.204) (end 116.082764 75.204) (width 0.25) (layer "F.Cu") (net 3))
 (segment (start 116.367 78.204) (end 117.348 79.185) (width 0.25) (layer "F.Cu") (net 1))
 (segment (start 115.44 78.204) (end 116.367 78.204) (width 0.25) (layer "F.Cu") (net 1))
 (via (at 118.872 74.676) (size 0.6) (drill 0.3) (layers "F.Cu" "B.Cu") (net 7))
 (via (at 125.73 78.74) (size 0.6) (drill 0.3) (layers "F.Cu" "B.Cu") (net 7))
 (via (at 118.872 73.914) (size 0.6) (drill 0.3) (layers "F.Cu" "B.Cu") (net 7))
 (via (at 122.682 77.724) (size 0.6) (drill 0.3) (layers "F.Cu" "B.Cu") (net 7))
 (via (at 122.682 78.74) (size 0.6) (drill 0.3) (layers "F.Cu" "B.Cu") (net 7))
 (via (at 118.872 78.994) (size 0.6) (drill 0.3) (layers "F.Cu" "B.Cu") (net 7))
 (via (at 118.872 78.232) (size 0.6) (drill 0.3) (layers "F.Cu" "B.Cu") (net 7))
 (via (at 125.73 77.724) (size 0.6) (drill 0.3) (layers "F.Cu" "B.Cu") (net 7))
 (segment (start 118.872 78.232) (end 118.872 74.676) (width 0.8) (layer "B.Cu") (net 7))
 (segment (start 118.872 74.676) (end 118.872 73.914) (width 0.8) (layer "B.Cu") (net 7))
 (segment (start 120.65 78.232) (end 124.206 78.232) (width 0.8) (layer "B.Cu") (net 7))
 (segment (start 118.872 78.994) (end 118.872 78.232) (width 0.8) (layer "B.Cu") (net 7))
 (segment (start 119.888 78.994) (end 120.65 78.232) (width 0.8) (layer "B.Cu") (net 7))
 (segment (start 118.872 78.994) (end 119.888 78.994) (width 0.8) (layer "B.Cu") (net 7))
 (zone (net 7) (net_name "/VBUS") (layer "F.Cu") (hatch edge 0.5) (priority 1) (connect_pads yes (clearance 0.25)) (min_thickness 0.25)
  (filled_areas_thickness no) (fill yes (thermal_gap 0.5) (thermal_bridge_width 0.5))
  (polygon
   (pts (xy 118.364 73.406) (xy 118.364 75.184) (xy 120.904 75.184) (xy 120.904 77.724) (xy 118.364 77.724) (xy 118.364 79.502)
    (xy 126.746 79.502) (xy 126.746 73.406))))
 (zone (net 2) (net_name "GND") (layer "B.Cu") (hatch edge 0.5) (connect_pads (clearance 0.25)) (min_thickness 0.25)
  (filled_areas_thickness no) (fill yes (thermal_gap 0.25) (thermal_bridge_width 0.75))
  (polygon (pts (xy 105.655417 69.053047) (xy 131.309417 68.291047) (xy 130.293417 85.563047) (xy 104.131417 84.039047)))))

